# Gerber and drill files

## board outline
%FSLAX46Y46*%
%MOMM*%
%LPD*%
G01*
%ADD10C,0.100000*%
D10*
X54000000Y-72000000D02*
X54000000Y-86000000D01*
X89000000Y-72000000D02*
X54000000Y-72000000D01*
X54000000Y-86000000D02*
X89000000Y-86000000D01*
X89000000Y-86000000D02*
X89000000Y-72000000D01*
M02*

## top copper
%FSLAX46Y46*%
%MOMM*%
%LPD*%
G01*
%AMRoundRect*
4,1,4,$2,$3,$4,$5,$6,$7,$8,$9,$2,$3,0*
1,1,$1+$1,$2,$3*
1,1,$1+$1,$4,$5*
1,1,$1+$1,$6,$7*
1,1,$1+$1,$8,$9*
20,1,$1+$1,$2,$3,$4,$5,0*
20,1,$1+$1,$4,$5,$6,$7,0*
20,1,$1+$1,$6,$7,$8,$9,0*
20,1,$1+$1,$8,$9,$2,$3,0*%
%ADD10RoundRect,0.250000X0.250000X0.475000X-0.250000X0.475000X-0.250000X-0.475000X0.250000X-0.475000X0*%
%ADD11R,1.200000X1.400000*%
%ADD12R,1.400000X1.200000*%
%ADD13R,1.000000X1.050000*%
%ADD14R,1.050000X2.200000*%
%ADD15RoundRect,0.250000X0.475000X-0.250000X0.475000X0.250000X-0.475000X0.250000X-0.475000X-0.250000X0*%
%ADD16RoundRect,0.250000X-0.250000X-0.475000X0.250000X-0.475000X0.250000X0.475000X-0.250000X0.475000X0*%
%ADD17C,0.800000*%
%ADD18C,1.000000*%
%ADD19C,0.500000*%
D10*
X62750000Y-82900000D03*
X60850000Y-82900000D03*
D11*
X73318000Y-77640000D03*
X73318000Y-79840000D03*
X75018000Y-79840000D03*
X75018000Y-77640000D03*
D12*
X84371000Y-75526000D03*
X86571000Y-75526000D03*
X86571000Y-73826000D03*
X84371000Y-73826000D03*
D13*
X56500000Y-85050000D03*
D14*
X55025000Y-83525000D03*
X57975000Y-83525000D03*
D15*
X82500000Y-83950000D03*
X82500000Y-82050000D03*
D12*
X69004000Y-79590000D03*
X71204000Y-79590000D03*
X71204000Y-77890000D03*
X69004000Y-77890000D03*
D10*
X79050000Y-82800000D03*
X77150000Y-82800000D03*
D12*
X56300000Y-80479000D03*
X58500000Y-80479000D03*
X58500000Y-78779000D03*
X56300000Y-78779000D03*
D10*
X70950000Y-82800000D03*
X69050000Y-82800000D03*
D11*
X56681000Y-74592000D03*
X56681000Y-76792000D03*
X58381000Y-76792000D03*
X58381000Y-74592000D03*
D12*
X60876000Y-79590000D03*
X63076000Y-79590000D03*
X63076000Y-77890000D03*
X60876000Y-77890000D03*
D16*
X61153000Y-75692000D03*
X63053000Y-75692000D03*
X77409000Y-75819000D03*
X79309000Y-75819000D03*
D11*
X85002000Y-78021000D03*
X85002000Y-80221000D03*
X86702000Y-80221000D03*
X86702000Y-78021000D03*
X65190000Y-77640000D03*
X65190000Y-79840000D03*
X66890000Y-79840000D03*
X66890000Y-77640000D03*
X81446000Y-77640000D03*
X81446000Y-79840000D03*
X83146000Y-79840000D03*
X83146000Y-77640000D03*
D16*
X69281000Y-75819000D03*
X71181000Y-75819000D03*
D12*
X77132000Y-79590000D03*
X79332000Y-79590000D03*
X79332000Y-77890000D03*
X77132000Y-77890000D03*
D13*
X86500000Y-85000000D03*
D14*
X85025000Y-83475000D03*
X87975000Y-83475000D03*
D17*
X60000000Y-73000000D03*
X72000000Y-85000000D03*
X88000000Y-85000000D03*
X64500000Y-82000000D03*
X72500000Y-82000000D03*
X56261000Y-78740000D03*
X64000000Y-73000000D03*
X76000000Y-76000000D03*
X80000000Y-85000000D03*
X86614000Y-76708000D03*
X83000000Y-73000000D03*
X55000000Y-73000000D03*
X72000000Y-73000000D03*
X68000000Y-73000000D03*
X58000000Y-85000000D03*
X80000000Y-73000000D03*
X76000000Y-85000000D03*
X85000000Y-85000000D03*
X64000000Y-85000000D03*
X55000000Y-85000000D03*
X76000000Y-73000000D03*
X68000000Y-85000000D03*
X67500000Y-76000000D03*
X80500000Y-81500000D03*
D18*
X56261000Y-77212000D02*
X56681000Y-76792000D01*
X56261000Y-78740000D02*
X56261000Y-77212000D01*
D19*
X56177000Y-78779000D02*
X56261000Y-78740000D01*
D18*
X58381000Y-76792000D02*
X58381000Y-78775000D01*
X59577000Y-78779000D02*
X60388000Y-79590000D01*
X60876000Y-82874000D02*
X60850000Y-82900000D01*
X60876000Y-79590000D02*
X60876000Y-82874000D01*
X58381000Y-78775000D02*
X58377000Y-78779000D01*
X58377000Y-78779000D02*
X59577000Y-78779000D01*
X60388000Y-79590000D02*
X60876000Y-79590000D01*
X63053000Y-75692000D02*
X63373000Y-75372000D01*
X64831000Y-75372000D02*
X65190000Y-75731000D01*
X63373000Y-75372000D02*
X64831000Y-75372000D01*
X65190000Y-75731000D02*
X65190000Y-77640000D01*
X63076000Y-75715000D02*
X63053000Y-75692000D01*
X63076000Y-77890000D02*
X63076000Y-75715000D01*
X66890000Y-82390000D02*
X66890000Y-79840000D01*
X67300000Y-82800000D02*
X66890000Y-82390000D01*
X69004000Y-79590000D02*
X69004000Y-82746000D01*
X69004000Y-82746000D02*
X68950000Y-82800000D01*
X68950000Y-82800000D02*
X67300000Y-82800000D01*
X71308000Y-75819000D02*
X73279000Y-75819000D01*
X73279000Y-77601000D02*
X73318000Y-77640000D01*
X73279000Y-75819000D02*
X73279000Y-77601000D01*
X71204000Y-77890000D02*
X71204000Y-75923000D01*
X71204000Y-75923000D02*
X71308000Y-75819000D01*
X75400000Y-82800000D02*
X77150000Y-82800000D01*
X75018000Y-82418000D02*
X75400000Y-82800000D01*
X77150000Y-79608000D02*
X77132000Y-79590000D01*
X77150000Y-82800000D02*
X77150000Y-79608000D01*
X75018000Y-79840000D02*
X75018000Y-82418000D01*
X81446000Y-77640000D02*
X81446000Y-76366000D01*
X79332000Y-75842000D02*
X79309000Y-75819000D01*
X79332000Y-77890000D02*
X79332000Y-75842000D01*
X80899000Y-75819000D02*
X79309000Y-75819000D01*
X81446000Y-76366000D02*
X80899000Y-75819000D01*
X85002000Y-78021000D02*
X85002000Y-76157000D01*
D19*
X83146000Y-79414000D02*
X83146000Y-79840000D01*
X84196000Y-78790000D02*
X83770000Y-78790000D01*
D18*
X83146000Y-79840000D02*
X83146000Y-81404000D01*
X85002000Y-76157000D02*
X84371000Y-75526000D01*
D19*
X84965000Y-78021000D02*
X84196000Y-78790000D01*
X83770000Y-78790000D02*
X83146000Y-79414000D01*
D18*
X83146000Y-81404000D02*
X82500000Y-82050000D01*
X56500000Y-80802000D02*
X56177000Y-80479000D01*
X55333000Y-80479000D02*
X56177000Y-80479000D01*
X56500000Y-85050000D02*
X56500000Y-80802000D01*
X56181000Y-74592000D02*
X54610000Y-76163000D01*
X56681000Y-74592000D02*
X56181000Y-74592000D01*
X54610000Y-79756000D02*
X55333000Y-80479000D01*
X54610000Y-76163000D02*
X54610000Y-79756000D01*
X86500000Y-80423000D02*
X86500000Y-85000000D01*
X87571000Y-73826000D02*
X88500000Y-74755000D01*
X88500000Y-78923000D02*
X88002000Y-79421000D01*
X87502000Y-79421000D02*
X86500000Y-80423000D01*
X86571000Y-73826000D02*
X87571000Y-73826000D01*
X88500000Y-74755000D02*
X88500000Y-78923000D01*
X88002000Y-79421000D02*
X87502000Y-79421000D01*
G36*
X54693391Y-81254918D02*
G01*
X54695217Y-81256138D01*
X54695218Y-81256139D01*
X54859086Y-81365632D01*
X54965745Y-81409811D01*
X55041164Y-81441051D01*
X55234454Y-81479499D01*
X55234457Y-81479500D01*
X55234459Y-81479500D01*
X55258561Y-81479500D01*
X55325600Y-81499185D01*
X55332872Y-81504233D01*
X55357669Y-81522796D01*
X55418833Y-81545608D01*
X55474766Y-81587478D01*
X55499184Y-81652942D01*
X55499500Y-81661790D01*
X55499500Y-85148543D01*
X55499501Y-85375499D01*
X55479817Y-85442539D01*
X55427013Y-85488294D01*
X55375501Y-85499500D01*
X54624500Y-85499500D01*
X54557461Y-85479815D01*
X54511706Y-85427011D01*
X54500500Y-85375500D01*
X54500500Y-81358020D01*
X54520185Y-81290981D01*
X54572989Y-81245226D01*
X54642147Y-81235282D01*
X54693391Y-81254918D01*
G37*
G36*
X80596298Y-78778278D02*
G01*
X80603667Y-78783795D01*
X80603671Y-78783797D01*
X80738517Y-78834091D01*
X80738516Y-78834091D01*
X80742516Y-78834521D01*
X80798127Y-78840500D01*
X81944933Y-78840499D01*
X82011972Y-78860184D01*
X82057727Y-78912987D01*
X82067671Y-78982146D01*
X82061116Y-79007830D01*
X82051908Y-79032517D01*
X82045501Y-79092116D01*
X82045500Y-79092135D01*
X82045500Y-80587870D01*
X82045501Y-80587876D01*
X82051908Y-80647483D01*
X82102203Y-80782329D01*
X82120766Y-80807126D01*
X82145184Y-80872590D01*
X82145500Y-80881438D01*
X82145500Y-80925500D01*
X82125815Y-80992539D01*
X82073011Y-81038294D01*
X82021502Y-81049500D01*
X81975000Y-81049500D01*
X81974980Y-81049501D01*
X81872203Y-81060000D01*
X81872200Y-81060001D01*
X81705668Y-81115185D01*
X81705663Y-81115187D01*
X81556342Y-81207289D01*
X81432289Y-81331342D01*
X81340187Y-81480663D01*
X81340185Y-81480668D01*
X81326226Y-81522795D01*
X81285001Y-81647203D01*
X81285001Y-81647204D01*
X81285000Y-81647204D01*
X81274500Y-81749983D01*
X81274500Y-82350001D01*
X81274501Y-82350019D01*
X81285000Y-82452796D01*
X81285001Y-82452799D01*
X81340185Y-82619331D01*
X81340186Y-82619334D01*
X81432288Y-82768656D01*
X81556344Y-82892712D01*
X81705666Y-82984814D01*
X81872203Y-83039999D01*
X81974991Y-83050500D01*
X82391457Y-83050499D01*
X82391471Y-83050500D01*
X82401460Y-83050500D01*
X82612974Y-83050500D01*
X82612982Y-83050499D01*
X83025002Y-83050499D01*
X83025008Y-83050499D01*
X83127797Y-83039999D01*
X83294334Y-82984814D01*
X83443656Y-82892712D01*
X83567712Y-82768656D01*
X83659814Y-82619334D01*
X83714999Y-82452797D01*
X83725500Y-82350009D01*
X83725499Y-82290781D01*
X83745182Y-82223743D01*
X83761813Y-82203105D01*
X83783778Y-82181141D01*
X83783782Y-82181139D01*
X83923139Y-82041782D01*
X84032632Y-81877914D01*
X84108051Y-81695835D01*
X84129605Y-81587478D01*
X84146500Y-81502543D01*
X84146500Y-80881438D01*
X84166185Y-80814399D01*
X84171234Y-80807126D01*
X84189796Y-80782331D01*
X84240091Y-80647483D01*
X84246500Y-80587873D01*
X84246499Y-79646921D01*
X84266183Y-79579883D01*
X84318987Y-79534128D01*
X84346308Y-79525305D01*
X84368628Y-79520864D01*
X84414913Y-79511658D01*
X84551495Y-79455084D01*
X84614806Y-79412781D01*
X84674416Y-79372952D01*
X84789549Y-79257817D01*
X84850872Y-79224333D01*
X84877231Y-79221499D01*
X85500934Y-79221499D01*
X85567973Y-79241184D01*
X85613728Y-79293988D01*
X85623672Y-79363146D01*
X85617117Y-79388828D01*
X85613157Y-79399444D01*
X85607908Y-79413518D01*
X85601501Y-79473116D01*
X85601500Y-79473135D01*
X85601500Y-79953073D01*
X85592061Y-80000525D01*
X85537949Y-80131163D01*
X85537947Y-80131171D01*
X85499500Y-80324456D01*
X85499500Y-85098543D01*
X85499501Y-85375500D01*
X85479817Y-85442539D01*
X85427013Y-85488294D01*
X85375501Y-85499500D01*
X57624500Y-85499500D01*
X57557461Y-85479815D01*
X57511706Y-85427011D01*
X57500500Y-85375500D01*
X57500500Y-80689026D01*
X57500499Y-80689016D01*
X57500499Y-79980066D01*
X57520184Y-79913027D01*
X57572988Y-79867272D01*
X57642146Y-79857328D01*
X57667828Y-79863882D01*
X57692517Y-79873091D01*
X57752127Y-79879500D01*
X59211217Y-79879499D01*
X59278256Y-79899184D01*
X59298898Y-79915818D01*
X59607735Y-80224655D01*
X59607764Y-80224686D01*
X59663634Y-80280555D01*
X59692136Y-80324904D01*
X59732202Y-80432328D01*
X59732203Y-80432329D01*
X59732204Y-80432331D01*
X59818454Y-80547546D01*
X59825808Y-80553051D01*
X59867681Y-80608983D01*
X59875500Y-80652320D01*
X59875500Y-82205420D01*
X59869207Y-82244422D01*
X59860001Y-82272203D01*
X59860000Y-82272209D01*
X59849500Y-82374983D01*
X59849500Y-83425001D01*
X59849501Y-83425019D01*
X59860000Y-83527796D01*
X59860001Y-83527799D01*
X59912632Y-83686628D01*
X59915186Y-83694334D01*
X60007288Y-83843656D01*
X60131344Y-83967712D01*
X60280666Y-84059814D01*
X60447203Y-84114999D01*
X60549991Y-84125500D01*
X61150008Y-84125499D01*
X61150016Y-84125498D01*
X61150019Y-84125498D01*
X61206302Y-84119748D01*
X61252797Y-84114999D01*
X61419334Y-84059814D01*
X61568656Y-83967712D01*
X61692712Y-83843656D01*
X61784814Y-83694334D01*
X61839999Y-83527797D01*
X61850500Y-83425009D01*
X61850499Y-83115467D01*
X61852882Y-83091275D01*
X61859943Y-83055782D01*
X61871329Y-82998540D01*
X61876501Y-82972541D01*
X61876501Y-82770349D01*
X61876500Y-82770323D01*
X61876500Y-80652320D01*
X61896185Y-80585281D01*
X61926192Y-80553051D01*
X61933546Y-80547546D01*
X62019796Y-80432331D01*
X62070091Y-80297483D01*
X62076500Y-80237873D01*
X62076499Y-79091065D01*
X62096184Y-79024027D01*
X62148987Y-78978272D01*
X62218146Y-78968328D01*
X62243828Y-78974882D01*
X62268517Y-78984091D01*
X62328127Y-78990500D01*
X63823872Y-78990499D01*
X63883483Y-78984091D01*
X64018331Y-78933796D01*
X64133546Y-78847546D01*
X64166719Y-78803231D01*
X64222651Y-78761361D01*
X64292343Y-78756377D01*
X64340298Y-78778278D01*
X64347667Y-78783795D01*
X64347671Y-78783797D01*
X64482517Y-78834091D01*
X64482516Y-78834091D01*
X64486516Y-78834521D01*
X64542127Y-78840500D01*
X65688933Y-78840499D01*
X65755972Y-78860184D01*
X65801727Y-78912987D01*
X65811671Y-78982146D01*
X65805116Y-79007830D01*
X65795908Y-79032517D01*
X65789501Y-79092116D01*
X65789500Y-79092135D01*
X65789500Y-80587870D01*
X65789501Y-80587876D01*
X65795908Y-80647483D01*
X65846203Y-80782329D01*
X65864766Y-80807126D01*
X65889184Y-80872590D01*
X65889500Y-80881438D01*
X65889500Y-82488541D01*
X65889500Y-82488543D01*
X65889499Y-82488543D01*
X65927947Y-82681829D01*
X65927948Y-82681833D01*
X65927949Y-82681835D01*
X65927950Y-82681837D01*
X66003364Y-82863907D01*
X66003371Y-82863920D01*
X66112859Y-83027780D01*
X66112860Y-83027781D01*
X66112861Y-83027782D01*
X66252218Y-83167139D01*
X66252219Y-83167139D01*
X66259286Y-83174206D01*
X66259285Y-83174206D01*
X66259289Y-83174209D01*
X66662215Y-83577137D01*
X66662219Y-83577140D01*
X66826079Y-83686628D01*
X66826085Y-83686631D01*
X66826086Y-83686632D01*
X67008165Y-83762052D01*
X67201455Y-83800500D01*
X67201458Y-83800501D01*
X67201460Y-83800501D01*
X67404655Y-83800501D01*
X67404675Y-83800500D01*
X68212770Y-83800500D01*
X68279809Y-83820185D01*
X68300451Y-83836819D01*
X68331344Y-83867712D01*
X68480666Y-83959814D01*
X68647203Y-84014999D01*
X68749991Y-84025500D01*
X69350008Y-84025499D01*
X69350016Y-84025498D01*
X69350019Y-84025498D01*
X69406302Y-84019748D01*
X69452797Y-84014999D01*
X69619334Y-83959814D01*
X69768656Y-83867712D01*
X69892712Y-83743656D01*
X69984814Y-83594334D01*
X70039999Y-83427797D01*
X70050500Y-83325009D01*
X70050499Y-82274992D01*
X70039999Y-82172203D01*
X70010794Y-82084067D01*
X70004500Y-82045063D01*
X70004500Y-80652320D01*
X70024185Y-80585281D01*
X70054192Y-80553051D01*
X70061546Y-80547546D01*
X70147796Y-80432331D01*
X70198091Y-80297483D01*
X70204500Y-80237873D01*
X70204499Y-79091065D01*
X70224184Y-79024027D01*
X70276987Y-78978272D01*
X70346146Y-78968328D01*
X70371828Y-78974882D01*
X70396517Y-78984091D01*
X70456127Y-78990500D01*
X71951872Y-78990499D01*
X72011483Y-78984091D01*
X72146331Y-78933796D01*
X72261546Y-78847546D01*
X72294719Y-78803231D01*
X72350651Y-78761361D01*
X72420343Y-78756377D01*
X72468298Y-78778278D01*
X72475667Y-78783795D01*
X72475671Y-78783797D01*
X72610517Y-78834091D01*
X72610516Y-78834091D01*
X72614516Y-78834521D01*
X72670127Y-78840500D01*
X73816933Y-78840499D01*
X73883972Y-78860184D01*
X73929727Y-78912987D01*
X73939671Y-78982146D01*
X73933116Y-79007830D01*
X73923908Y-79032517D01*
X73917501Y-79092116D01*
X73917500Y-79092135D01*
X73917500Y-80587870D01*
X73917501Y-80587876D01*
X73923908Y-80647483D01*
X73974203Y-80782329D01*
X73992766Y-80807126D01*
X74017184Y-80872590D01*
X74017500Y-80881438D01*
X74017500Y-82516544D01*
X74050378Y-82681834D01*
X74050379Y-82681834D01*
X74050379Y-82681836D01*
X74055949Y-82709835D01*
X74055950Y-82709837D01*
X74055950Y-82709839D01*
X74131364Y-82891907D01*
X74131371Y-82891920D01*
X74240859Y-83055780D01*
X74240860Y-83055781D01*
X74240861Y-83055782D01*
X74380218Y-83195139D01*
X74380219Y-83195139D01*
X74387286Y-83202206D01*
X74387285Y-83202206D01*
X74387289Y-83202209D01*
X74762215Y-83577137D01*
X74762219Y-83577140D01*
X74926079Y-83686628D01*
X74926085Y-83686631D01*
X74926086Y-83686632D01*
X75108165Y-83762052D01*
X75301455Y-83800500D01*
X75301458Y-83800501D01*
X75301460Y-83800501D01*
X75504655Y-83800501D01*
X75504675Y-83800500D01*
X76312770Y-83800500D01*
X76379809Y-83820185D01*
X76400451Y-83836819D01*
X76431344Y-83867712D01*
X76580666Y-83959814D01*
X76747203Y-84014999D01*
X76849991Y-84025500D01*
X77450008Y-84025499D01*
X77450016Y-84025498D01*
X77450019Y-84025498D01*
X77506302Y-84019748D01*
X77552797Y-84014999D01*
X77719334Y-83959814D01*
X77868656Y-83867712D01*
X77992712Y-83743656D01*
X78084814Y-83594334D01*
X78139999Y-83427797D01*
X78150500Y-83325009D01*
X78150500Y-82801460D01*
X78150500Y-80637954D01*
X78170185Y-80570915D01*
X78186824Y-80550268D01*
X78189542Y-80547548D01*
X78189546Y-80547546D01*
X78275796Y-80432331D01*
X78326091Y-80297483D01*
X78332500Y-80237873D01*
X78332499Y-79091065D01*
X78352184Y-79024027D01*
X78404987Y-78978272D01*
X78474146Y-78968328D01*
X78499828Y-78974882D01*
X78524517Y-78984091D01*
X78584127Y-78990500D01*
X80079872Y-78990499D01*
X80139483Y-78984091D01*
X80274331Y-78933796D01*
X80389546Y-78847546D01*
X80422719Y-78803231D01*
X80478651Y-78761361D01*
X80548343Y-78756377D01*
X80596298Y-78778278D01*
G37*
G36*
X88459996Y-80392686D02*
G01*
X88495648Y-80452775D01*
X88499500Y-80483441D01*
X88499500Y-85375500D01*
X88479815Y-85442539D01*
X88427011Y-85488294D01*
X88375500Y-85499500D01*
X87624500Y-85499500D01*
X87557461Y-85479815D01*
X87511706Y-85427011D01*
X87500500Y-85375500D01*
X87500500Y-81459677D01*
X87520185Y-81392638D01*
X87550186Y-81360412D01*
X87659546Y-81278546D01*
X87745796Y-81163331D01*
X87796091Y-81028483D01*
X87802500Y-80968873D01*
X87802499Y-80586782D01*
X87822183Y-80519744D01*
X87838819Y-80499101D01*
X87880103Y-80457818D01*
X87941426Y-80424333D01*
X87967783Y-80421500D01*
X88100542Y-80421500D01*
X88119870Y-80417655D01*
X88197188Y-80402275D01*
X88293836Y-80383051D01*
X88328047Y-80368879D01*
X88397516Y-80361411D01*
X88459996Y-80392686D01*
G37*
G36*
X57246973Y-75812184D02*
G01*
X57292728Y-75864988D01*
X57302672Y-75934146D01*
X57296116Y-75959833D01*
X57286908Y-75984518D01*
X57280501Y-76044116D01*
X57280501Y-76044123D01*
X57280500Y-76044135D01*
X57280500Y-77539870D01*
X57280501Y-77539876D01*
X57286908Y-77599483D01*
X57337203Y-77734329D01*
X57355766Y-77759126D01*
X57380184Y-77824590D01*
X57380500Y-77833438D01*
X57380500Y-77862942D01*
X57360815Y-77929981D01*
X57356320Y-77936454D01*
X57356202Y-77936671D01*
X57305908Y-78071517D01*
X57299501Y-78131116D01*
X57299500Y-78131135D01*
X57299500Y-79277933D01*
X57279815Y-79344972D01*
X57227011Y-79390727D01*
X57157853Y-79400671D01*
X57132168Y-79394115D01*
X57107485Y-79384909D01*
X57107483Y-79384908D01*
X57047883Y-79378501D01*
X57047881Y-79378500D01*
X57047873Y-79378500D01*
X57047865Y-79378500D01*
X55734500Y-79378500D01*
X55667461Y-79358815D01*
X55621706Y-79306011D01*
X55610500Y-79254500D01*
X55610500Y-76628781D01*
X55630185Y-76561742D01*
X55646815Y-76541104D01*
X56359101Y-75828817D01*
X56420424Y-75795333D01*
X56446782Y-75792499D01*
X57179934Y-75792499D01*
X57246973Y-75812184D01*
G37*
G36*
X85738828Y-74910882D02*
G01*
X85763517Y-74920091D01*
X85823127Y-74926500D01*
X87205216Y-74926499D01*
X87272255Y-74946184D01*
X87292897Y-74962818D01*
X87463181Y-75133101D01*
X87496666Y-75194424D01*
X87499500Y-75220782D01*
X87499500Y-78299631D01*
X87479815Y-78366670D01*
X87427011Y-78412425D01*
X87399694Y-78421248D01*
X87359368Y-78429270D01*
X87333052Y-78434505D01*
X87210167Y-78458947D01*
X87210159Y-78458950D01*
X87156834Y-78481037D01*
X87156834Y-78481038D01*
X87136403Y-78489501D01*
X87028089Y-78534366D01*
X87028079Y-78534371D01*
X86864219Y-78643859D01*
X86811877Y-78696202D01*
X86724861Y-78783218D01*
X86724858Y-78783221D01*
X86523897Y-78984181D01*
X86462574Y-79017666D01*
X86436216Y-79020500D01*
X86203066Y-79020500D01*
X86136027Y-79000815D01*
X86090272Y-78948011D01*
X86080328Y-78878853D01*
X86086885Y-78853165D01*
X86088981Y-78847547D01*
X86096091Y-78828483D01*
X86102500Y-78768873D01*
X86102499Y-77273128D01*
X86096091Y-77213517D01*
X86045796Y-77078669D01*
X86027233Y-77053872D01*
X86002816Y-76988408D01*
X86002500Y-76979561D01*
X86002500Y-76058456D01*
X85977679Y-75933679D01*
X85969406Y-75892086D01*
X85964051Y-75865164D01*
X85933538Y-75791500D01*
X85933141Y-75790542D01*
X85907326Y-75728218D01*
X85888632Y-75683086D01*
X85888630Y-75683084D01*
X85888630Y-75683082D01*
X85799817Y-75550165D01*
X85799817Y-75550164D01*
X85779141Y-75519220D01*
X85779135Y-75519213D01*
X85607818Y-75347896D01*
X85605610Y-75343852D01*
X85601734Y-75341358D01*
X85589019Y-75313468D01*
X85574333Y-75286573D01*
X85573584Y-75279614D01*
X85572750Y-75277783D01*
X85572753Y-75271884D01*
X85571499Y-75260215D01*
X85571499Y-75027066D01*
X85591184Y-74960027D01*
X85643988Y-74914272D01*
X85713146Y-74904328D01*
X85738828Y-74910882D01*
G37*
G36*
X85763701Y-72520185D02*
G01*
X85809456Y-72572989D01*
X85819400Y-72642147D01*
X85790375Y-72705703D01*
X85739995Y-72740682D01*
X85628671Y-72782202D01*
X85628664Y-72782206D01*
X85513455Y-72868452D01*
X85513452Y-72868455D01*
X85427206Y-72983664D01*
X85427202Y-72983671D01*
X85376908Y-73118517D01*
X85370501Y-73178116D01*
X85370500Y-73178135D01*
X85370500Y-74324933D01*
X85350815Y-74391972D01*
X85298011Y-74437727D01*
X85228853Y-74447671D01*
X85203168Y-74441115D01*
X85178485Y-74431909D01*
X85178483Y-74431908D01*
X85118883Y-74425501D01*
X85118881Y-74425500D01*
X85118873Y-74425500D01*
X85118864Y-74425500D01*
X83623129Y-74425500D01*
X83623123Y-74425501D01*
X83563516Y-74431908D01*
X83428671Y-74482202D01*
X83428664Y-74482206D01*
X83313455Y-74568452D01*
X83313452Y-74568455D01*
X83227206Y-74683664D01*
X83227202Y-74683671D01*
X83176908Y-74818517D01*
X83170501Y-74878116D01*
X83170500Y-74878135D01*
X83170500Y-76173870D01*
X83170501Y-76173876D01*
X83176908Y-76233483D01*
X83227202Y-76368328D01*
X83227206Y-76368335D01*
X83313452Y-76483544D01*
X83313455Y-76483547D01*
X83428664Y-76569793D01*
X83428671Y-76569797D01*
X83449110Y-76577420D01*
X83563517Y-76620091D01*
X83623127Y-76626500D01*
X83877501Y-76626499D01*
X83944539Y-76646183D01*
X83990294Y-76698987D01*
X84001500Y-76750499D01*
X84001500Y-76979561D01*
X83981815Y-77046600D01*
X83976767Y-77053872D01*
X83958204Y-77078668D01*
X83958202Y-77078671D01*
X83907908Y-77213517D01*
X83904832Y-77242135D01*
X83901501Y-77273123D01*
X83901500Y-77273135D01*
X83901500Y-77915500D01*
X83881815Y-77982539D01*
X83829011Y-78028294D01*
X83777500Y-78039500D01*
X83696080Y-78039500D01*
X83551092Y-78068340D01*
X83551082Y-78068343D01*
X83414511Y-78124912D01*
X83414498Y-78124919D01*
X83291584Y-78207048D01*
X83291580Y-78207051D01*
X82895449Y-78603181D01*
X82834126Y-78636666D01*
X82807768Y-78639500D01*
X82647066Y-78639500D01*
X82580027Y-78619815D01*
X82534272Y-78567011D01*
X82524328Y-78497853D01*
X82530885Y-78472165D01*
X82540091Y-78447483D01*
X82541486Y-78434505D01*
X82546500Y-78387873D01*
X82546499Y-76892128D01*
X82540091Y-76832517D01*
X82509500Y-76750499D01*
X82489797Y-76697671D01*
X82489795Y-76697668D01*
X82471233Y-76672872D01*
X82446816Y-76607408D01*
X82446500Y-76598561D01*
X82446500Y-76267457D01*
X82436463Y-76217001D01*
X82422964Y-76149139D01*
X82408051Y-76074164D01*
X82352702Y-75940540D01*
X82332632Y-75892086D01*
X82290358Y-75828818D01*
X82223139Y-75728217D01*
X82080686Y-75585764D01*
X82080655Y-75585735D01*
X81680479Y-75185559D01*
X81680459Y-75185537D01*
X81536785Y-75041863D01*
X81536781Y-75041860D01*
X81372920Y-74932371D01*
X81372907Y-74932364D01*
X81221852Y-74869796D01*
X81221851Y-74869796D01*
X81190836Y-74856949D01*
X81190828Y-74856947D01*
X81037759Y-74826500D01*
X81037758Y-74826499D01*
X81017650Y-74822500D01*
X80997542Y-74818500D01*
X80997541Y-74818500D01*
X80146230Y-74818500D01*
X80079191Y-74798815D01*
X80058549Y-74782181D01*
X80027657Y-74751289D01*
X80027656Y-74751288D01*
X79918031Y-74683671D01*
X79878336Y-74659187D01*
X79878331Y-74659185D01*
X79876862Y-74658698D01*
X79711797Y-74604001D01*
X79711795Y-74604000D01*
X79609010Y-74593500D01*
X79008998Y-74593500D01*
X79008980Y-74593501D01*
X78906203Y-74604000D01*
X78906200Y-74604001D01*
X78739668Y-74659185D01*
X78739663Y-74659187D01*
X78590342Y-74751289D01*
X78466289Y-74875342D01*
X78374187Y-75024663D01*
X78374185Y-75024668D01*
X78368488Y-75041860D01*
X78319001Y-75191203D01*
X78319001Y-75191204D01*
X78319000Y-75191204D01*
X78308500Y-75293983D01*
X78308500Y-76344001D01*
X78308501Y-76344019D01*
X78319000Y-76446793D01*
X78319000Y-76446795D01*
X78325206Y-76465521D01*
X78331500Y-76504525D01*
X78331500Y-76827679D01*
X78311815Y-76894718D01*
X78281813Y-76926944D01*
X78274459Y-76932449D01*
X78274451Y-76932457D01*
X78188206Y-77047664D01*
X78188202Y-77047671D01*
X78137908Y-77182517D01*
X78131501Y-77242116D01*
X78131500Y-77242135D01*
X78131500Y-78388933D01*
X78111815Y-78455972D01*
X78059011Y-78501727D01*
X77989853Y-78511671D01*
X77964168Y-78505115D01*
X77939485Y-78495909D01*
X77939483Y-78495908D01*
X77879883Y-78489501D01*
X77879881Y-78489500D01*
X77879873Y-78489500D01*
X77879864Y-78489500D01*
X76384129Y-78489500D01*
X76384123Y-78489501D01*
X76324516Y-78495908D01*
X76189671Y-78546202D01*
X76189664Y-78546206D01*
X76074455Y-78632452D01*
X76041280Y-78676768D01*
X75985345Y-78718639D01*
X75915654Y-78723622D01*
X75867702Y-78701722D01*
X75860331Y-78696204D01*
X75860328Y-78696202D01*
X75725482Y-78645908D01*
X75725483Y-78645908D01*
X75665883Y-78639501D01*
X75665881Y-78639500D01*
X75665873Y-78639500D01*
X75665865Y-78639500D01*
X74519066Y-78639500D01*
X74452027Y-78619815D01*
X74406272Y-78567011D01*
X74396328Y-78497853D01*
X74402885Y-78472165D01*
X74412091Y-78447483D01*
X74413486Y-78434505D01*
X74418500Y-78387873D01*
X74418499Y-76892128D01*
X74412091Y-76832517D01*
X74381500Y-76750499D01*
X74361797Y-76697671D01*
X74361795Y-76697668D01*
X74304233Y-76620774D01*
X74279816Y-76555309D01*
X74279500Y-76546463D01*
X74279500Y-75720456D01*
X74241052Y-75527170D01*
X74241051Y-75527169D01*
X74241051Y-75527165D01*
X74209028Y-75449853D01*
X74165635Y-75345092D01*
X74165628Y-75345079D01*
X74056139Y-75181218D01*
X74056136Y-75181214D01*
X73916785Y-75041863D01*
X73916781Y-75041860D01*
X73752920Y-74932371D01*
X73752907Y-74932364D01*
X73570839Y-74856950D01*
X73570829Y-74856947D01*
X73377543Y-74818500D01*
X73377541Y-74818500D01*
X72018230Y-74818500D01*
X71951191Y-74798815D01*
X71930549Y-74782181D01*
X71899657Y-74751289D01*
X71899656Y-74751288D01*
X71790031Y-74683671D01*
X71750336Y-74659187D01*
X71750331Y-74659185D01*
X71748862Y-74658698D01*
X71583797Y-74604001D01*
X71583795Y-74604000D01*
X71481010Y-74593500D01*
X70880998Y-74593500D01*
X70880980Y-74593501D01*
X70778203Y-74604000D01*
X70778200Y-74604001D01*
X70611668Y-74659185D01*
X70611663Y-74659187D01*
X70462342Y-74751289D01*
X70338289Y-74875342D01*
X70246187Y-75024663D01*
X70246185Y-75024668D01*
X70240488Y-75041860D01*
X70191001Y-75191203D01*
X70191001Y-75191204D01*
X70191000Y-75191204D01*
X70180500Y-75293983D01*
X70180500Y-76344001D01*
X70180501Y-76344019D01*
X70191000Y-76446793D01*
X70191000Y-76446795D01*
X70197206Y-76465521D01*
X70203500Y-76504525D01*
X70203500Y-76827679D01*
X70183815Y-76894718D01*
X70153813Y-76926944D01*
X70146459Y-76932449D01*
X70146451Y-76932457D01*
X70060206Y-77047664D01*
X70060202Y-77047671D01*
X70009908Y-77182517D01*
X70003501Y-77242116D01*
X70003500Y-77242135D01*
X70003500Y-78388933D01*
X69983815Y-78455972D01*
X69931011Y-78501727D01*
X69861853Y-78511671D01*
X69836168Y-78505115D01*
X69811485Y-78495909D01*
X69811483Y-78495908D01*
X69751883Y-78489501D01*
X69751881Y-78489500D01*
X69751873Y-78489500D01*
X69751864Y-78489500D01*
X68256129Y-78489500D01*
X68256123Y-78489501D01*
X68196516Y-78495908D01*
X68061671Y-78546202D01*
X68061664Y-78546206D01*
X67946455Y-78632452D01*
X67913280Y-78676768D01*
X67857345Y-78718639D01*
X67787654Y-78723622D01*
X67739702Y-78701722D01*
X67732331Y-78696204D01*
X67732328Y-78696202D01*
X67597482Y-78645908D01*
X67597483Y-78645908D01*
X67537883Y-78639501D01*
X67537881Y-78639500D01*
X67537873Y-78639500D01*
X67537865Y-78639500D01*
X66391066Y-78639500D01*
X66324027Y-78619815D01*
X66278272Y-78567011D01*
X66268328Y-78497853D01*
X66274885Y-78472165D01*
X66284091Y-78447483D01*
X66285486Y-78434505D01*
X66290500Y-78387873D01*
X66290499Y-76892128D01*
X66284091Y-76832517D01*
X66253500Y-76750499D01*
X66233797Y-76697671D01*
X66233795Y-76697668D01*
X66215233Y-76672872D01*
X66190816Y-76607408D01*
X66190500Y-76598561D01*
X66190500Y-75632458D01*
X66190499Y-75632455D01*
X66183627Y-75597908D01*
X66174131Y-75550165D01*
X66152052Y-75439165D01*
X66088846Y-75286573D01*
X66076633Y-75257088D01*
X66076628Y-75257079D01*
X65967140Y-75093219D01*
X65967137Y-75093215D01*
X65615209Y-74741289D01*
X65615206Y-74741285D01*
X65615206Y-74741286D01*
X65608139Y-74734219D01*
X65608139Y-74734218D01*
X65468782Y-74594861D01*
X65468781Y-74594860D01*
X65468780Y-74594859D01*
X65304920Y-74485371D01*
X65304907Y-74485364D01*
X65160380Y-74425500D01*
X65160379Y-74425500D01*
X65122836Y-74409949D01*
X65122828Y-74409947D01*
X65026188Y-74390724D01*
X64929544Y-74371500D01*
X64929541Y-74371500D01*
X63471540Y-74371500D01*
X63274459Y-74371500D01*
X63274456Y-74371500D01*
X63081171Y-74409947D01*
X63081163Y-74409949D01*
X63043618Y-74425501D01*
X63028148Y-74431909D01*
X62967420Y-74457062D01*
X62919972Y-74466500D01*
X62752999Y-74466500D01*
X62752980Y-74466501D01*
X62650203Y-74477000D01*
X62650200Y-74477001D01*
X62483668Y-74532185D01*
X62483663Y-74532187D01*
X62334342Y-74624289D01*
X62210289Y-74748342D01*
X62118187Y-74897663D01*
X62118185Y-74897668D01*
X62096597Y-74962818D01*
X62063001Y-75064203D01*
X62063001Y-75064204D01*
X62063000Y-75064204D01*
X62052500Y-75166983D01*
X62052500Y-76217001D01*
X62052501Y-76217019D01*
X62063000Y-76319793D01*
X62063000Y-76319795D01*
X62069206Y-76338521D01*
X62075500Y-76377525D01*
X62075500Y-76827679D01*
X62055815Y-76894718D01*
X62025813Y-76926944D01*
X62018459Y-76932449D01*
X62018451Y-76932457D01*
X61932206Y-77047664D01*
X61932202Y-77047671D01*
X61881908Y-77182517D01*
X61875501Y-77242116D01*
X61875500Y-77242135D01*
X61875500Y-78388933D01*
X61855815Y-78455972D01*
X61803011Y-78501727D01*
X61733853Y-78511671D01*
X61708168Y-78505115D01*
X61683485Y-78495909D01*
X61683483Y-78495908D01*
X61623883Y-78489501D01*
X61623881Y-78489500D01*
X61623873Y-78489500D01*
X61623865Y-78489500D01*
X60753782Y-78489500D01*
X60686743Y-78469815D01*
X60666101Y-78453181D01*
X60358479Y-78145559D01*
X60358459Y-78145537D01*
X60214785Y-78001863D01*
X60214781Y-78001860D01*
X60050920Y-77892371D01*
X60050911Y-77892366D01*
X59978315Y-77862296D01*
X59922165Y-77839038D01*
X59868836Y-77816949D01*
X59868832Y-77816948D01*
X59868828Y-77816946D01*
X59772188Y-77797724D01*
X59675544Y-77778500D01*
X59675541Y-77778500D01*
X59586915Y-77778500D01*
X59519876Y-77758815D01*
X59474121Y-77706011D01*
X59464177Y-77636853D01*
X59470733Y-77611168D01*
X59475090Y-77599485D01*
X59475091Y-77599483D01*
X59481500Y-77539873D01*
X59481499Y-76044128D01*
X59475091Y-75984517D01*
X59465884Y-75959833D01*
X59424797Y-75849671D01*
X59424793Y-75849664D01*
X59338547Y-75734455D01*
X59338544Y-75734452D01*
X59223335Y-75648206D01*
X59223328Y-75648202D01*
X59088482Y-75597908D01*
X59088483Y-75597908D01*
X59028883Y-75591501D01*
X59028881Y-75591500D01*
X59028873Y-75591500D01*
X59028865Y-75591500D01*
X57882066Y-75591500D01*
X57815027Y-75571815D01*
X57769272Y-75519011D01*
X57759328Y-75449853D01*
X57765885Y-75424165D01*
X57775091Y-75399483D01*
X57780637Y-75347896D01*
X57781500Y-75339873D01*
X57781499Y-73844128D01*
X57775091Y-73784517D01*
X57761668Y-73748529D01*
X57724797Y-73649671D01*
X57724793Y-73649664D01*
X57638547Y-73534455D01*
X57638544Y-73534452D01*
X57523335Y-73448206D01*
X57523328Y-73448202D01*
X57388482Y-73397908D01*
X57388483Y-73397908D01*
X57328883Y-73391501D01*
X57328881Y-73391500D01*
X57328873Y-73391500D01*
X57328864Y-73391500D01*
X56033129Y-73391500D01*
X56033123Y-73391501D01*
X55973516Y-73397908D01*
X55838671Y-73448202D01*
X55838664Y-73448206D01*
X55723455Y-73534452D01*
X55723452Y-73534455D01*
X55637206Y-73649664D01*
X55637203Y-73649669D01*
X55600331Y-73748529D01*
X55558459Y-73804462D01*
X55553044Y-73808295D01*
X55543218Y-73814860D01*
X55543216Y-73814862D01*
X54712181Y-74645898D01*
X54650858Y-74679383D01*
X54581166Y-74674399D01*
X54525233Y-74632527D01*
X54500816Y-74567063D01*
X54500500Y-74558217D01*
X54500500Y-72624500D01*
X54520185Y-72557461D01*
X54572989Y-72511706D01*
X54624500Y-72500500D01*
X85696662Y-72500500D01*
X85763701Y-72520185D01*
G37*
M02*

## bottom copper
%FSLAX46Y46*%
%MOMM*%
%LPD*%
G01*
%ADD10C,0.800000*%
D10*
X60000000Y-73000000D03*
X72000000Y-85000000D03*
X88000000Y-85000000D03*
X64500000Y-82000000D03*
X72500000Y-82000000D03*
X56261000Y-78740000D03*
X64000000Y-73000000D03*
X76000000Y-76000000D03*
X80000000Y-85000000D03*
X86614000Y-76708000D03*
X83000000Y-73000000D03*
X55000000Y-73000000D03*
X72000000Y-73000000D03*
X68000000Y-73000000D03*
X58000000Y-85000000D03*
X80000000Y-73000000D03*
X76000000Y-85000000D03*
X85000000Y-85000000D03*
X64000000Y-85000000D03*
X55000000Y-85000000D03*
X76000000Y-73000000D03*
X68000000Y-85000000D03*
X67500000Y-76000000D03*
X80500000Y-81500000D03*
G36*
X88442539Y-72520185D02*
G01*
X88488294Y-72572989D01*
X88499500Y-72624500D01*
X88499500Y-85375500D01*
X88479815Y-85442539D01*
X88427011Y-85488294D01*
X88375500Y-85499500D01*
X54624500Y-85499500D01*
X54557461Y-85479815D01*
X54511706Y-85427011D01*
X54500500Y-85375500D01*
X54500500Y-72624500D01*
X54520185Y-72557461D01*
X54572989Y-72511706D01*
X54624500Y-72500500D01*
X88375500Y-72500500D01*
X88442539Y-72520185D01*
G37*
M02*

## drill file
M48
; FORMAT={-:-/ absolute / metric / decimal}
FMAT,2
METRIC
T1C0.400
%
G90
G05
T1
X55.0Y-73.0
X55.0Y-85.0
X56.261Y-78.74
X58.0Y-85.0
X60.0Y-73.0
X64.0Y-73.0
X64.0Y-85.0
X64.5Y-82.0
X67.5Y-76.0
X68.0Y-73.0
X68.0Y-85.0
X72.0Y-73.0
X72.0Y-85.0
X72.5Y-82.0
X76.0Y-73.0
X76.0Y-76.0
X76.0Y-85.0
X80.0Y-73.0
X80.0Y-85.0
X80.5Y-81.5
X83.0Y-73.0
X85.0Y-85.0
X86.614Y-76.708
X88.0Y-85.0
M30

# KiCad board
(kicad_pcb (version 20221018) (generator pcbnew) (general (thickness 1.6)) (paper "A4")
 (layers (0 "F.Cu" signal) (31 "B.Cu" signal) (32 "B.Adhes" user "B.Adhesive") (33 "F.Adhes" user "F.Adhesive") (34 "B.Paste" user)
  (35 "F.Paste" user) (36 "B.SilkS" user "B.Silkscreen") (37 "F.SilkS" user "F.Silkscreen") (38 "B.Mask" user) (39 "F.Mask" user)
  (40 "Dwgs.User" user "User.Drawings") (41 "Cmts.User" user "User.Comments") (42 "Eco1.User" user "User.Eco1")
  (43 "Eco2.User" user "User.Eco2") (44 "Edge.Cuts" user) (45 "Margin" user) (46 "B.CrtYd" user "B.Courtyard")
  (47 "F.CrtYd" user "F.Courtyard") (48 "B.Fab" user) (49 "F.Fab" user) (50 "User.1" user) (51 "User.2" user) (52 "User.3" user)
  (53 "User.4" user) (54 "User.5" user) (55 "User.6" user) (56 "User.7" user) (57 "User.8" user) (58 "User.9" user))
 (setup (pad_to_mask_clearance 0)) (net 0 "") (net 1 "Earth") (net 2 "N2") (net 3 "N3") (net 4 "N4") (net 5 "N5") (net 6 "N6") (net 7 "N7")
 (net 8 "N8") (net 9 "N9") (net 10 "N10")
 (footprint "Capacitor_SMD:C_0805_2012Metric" (layer "F.Cu") (at 61.8 82.9 180)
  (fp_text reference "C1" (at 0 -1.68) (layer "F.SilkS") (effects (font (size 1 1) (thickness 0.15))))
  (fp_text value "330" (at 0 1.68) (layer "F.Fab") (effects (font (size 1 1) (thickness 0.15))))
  (pad "1" smd roundrect (at -0.95 0 180) (size 1 1.45) (layers "F.Cu" "F.Paste" "F.Mask") (roundrect_rratio 0.25) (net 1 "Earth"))
  (pad "2" smd roundrect (at 0.95 0 180) (size 1 1.45) (layers "F.Cu" "F.Paste" "F.Mask") (roundrect_rratio 0.25) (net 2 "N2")))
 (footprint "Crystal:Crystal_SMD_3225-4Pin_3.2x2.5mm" (layer "F.Cu") (at 74.168 78.74 -90)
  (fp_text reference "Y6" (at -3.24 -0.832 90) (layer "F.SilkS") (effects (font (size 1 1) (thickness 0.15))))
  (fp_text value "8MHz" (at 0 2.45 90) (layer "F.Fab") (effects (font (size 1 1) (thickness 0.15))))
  (pad "1" smd rect (at -1.1 0.85 270) (size 1.4 1.2) (layers "F.Cu" "F.Paste" "F.Mask") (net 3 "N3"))
  (pad "2" smd rect (at 1.1 0.85 270) (size 1.4 1.2) (layers "F.Cu" "F.Paste" "F.Mask") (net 1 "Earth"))
  (pad "3" smd rect (at 1.1 -0.85 270) (size 1.4 1.2) (layers "F.Cu" "F.Paste" "F.Mask") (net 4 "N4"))
  (pad "4" smd rect (at -1.1 -0.85 270) (size 1.4 1.2) (layers "F.Cu" "F.Paste" "F.Mask") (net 1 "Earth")))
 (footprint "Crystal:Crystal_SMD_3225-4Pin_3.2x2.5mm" (layer "F.Cu") (at 85.471 74.676)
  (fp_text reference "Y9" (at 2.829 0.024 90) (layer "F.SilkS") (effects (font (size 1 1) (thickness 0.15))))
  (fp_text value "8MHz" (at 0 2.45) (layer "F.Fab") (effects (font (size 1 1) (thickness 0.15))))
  (pad "1" smd rect (at -1.1 0.85) (size 1.4 1.2) (layers "F.Cu" "F.Paste" "F.Mask") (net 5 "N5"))
  (pad "2" smd rect (at 1.1 0.85) (size 1.4 1.2) (layers "F.Cu" "F.Paste" "F.Mask") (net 1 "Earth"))
  (pad "3" smd rect (at 1.1 -0.85) (size 1.4 1.2) (layers "F.Cu" "F.Paste" "F.Mask") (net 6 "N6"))
  (pad "4" smd rect (at -1.1 -0.85) (size 1.4 1.2) (layers "F.Cu" "F.Paste" "F.Mask") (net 1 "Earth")))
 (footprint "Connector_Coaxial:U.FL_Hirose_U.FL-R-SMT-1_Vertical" (layer "F.Cu") (at 56.5 84 90)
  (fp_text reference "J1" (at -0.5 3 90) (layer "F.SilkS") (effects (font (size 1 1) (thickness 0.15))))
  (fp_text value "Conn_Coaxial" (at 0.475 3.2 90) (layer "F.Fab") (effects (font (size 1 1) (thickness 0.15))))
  (pad "1" smd rect (at -1.05 0 90) (size 1.05 1) (layers "F.Cu" "F.Paste" "F.Mask") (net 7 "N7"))
  (pad "2" smd rect (at 0.475 -1.475 90) (size 2.2 1.05) (layers "F.Cu" "F.Paste" "F.Mask") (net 1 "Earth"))
  (pad "2" smd rect (at 0.475 1.475 90) (size 2.2 1.05) (layers "F.Cu" "F.Paste" "F.Mask") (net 1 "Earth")))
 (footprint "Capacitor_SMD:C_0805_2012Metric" (layer "F.Cu") (at 82.5 83 90)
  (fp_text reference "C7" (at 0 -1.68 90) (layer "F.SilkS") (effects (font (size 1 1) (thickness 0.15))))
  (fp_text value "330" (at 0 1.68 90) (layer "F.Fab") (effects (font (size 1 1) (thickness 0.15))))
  (pad "1" smd roundrect (at -0.95 0 90) (size 1 1.45) (layers "F.Cu" "F.Paste" "F.Mask") (roundrect_rratio 0.25) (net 1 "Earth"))
  (pad "2" smd roundrect (at 0.95 0 90) (size 1 1.45) (layers "F.Cu" "F.Paste" "F.Mask") (roundrect_rratio 0.25) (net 5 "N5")))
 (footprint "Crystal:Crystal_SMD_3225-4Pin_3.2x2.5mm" (layer "F.Cu") (at 70.104 78.74)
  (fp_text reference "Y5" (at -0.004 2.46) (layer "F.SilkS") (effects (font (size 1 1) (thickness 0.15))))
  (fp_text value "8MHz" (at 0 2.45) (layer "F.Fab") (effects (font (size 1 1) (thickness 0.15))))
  (pad "1" smd rect (at -1.1 0.85) (size 1.4 1.2) (layers "F.Cu" "F.Paste" "F.Mask") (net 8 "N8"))
  (pad "2" smd rect (at 1.1 0.85) (size 1.4 1.2) (layers "F.Cu" "F.Paste" "F.Mask") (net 1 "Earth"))
  (pad "3" smd rect (at 1.1 -0.85) (size 1.4 1.2) (layers "F.Cu" "F.Paste" "F.Mask") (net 3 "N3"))
  (pad "4" smd rect (at -1.1 -0.85) (size 1.4 1.2) (layers "F.Cu" "F.Paste" "F.Mask") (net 1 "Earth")))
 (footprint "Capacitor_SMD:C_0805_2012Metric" (layer "F.Cu") (at 78.1 82.8 180)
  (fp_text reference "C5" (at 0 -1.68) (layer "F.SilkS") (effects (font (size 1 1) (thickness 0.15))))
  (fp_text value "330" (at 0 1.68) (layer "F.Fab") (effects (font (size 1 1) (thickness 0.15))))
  (pad "1" smd roundrect (at -0.95 0 180) (size 1 1.45) (layers "F.Cu" "F.Paste" "F.Mask") (roundrect_rratio 0.25) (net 1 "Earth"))
  (pad "2" smd roundrect (at 0.95 0 180) (size 1 1.45) (layers "F.Cu" "F.Paste" "F.Mask") (roundrect_rratio 0.25) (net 4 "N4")))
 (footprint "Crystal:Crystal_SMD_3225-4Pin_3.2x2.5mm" (layer "F.Cu") (at 57.4 79.629)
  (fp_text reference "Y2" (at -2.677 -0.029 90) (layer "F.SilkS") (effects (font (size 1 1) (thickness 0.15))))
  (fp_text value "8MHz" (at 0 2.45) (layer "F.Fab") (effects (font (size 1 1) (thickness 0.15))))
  (pad "1" smd rect (at -1.1 0.85) (size 1.4 1.2) (layers "F.Cu" "F.Paste" "F.Mask") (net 7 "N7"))
  (pad "2" smd rect (at 1.1 0.85) (size 1.4 1.2) (layers "F.Cu" "F.Paste" "F.Mask") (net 1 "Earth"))
  (pad "3" smd rect (at 1.1 -0.85) (size 1.4 1.2) (layers "F.Cu" "F.Paste" "F.Mask") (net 2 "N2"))
  (pad "4" smd rect (at -1.1 -0.85) (size 1.4 1.2) (layers "F.Cu" "F.Paste" "F.Mask") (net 1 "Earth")))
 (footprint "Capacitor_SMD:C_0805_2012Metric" (layer "F.Cu") (at 70 82.8 180)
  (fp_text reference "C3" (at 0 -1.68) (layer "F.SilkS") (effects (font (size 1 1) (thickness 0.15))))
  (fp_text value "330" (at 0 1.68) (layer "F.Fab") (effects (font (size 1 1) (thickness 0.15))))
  (pad "1" smd roundrect (at -0.95 0 180) (size 1 1.45) (layers "F.Cu" "F.Paste" "F.Mask") (roundrect_rratio 0.25) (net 1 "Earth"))
  (pad "2" smd roundrect (at 0.95 0 180) (size 1 1.45) (layers "F.Cu" "F.Paste" "F.Mask") (roundrect_rratio 0.25) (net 8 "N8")))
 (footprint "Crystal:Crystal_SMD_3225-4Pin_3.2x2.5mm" (layer "F.Cu") (at 57.531 75.692 -90)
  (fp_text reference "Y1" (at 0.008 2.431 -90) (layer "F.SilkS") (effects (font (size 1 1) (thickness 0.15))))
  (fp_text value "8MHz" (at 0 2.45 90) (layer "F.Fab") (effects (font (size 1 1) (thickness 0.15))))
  (pad "1" smd rect (at -1.1 0.85 270) (size 1.4 1.2) (layers "F.Cu" "F.Paste" "F.Mask") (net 7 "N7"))
  (pad "2" smd rect (at 1.1 0.85 270) (size 1.4 1.2) (layers "F.Cu" "F.Paste" "F.Mask") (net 1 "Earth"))
  (pad "3" smd rect (at 1.1 -0.85 270) (size 1.4 1.2) (layers "F.Cu" "F.Paste" "F.Mask") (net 2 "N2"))
  (pad "4" smd rect (at -1.1 -0.85 270) (size 1.4 1.2) (layers "F.Cu" "F.Paste" "F.Mask") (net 1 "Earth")))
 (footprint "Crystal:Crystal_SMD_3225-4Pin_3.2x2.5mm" (layer "F.Cu") (at 61.976 78.74)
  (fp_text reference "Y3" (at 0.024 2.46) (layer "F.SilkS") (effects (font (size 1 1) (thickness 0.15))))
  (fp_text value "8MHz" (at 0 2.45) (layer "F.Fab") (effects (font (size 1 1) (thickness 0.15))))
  (pad "1" smd rect (at -1.1 0.85) (size 1.4 1.2) (layers "F.Cu" "F.Paste" "F.Mask") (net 2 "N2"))
  (pad "2" smd rect (at 1.1 0.85) (size 1.4 1.2) (layers "F.Cu" "F.Paste" "F.Mask") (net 1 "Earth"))
  (pad "3" smd rect (at 1.1 -0.85) (size 1.4 1.2) (layers "F.Cu" "F.Paste" "F.Mask") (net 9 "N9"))
  (pad "4" smd rect (at -1.1 -0.85) (size 1.4 1.2) (layers "F.Cu" "F.Paste" "F.Mask") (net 1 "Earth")))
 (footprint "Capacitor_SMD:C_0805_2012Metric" (layer "F.Cu") (at 62.103 75.692)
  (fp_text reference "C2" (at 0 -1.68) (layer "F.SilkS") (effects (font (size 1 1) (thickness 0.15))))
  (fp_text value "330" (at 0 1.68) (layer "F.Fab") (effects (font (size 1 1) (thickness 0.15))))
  (pad "1" smd roundrect (at -0.95 0) (size 1 1.45) (layers "F.Cu" "F.Paste" "F.Mask") (roundrect_rratio 0.25) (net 1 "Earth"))
  (pad "2" smd roundrect (at 0.95 0) (size 1 1.45) (layers "F.Cu" "F.Paste" "F.Mask") (roundrect_rratio 0.25) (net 9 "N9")))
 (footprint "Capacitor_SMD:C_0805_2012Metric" (layer "F.Cu") (at 78.359 75.819)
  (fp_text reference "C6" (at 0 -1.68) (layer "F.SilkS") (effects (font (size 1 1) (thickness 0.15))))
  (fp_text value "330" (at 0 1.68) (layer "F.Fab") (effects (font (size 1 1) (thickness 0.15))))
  (pad "1" smd roundrect (at -0.95 0) (size 1 1.45) (layers "F.Cu" "F.Paste" "F.Mask") (roundrect_rratio 0.25) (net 1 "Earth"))
  (pad "2" smd roundrect (at 0.95 0) (size 1 1.45) (layers "F.Cu" "F.Paste" "F.Mask") (roundrect_rratio 0.25) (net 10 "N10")))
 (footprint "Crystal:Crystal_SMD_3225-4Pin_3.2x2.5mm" (layer "F.Cu") (at 85.852 79.121 -90)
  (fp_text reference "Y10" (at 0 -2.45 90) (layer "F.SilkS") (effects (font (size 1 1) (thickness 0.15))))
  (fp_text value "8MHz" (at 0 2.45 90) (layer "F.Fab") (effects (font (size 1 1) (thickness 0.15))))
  (pad "1" smd rect (at -1.1 0.85 270) (size 1.4 1.2) (layers "F.Cu" "F.Paste" "F.Mask") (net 5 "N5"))
  (pad "2" smd rect (at 1.1 0.85 270) (size 1.4 1.2) (layers "F.Cu" "F.Paste" "F.Mask") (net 1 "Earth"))
  (pad "3" smd rect (at 1.1 -0.85 270) (size 1.4 1.2) (layers "F.Cu" "F.Paste" "F.Mask") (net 6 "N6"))
  (pad "4" smd rect (at -1.1 -0.85 270) (size 1.4 1.2) (layers "F.Cu" "F.Paste" "F.Mask") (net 1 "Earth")))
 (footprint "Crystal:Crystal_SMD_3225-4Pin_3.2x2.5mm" (layer "F.Cu") (at 66.04 78.74 -90)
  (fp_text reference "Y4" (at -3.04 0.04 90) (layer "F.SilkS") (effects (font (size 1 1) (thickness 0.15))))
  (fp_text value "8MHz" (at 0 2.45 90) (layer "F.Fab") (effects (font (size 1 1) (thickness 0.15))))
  (pad "1" smd rect (at -1.1 0.85 270) (size 1.4 1.2) (layers "F.Cu" "F.Paste" "F.Mask") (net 9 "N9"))
  (pad "2" smd rect (at 1.1 0.85 270) (size 1.4 1.2) (layers "F.Cu" "F.Paste" "F.Mask") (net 1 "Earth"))
  (pad "3" smd rect (at 1.1 -0.85 270) (size 1.4 1.2) (layers "F.Cu" "F.Paste" "F.Mask") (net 8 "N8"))
  (pad "4" smd rect (at -1.1 -0.85 270) (size 1.4 1.2) (layers "F.Cu" "F.Paste" "F.Mask") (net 1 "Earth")))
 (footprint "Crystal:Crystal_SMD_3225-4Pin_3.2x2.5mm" (layer "F.Cu") (at 82.296 78.74 -90)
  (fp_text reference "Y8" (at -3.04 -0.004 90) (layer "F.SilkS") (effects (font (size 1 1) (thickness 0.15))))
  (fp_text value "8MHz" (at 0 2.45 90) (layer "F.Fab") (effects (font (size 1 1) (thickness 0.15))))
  (pad "1" smd rect (at -1.1 0.85 270) (size 1.4 1.2) (layers "F.Cu" "F.Paste" "F.Mask") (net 10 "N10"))
  (pad "2" smd rect (at 1.1 0.85 270) (size 1.4 1.2) (layers "F.Cu" "F.Paste" "F.Mask") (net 1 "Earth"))
  (pad "3" smd rect (at 1.1 -0.85 270) (size 1.4 1.2) (layers "F.Cu" "F.Paste" "F.Mask") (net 5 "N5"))
  (pad "4" smd rect (at -1.1 -0.85 270) (size 1.4 1.2) (layers "F.Cu" "F.Paste" "F.Mask") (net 1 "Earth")))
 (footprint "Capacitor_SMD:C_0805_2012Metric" (layer "F.Cu") (at 70.231 75.819)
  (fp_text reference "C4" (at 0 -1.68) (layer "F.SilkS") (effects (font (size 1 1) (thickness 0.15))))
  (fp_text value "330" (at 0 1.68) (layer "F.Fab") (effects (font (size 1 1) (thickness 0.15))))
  (pad "1" smd roundrect (at -0.95 0) (size 1 1.45) (layers "F.Cu" "F.Paste" "F.Mask") (roundrect_rratio 0.25) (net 1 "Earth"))
  (pad "2" smd roundrect (at 0.95 0) (size 1 1.45) (layers "F.Cu" "F.Paste" "F.Mask") (roundrect_rratio 0.25) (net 3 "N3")))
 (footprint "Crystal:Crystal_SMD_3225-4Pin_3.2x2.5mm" (layer "F.Cu") (at 78.232 78.74)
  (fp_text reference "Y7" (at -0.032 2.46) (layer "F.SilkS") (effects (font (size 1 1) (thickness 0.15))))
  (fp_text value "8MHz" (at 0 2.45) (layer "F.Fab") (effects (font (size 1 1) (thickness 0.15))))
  (pad "1" smd rect (at -1.1 0.85) (size 1.4 1.2) (layers "F.Cu" "F.Paste" "F.Mask") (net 4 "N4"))
  (pad "2" smd rect (at 1.1 0.85) (size 1.4 1.2) (layers "F.Cu" "F.Paste" "F.Mask") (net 1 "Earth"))
  (pad "3" smd rect (at 1.1 -0.85) (size 1.4 1.2) (layers "F.Cu" "F.Paste" "F.Mask") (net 10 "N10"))
  (pad "4" smd rect (at -1.1 -0.85) (size 1.4 1.2) (layers "F.Cu" "F.Paste" "F.Mask") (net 1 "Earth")))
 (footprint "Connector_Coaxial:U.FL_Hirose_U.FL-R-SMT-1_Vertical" (layer "F.Cu") (at 86.5 83.95 90)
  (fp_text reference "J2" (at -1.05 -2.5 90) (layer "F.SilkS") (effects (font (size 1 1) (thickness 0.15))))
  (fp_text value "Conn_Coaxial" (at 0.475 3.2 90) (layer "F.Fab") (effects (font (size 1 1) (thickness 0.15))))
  (pad "1" smd rect (at -1.05 0 90) (size 1.05 1) (layers "F.Cu" "F.Paste" "F.Mask") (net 6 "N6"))
  (pad "2" smd rect (at 0.475 -1.475 90) (size 2.2 1.05) (layers "F.Cu" "F.Paste" "F.Mask") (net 1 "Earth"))
  (pad "2" smd rect (at 0.475 1.475 90) (size 2.2 1.05) (layers "F.Cu" "F.Paste" "F.Mask") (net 1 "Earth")))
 (gr_line (start 54 72) (end 54 86) (stroke (width 0.1) (type default)) (layer "Edge.Cuts"))
 (gr_line (start 89 72) (end 54 72) (stroke (width 0.1) (type default)) (layer "Edge.Cuts"))
 (gr_line (start 54 86) (end 89 86) (stroke (width 0.1) (type default)) (layer "Edge.Cuts"))
 (gr_line (start 89 86) (end 89 72) (stroke (width 0.1) (type default)) (layer "Edge.Cuts"))
 (segment (start 56.261 77.212) (end 56.681 76.792) (width 1) (layer "F.Cu") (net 1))
 (segment (start 56.261 78.74) (end 56.261 77.212) (width 1) (layer "F.Cu") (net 1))
 (segment (start 56.177 78.779) (end 56.261 78.74) (width 0.5) (layer "F.Cu") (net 1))
 (via (at 60 73) (size 0.8) (drill 0.4) (layers "F.Cu" "B.Cu") (free) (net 1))
 (via (at 72 85) (size 0.8) (drill 0.4) (layers "F.Cu" "B.Cu") (free) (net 1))
 (via (at 88 85) (size 0.8) (drill 0.4) (layers "F.Cu" "B.Cu") (free) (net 1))
 (via (at 64.5 82) (size 0.8) (drill 0.4) (layers "F.Cu" "B.Cu") (free) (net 1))
 (via (at 72.5 82) (size 0.8) (drill 0.4) (layers "F.Cu" "B.Cu") (free) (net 1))
 (via (at 56.261 78.74) (size 0.8) (drill 0.4) (layers "F.Cu" "B.Cu") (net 1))
 (via (at 64 73) (size 0.8) (drill 0.4) (layers "F.Cu" "B.Cu") (free) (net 1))
 (via (at 76 76) (size 0.8) (drill 0.4) (layers "F.Cu" "B.Cu") (free) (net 1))
 (via (at 80 85) (size 0.8) (drill 0.4) (layers "F.Cu" "B.Cu") (free) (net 1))
 (via (at 86.614 76.708) (size 0.8) (drill 0.4) (layers "F.Cu" "B.Cu") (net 1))
 (via (at 83 73) (size 0.8) (drill 0.4) (layers "F.Cu" "B.Cu") (free) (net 1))
 (via (at 55 73) (size 0.8) (drill 0.4) (layers "F.Cu" "B.Cu") (free) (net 1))
 (via (at 72 73) (size 0.8) (drill 0.4) (layers "F.Cu" "B.Cu") (free) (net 1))
 (via (at 68 73) (size 0.8) (drill 0.4) (layers "F.Cu" "B.Cu") (free) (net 1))
 (via (at 58 85) (size 0.8) (drill 0.4) (layers "F.Cu" "B.Cu") (free) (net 1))
 (via (at 80 73) (size 0.8) (drill 0.4) (layers "F.Cu" "B.Cu") (free) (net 1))
 (via (at 76 85) (size 0.8) (drill 0.4) (layers "F.Cu" "B.Cu") (free) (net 1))
 (via (at 85 85) (size 0.8) (drill 0.4) (layers "F.Cu" "B.Cu") (free) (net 1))
 (via (at 64 85) (size 0.8) (drill 0.4) (layers "F.Cu" "B.Cu") (free) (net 1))
 (via (at 55 85) (size 0.8) (drill 0.4) (layers "F.Cu" "B.Cu") (free) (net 1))
 (via (at 76 73) (size 0.8) (drill 0.4) (layers "F.Cu" "B.Cu") (free) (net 1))
 (via (at 68 85) (size 0.8) (drill 0.4) (layers "F.Cu" "B.Cu") (free) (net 1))
 (via (at 67.5 76) (size 0.8) (drill 0.4) (layers "F.Cu" "B.Cu") (free) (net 1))
 (via (at 80.5 81.5) (size 0.8) (drill 0.4) (layers "F.Cu" "B.Cu") (free) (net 1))
 (segment (start 58.381 76.792) (end 58.381 78.775) (width 1) (layer "F.Cu") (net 2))
 (segment (start 59.577 78.779) (end 60.388 79.59) (width 1) (layer "F.Cu") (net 2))
 (segment (start 60.876 82.874) (end 60.85 82.9) (width 1) (layer "F.Cu") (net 2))
 (segment (start 60.876 79.59) (end 60.876 82.874) (width 1) (layer "F.Cu") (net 2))
 (segment (start 58.381 78.775) (end 58.377 78.779) (width 1) (layer "F.Cu") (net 2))
 (segment (start 58.377 78.779) (end 59.577 78.779) (width 1) (layer "F.Cu") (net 2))
 (segment (start 60.388 79.59) (end 60.876 79.59) (width 1) (layer "F.Cu") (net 2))
 (segment (start 63.053 75.692) (end 63.373 75.372) (width 1) (layer "F.Cu") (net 9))
 (segment (start 64.831 75.372) (end 65.19 75.731) (width 1) (layer "F.Cu") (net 9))
 (segment (start 63.373 75.372) (end 64.831 75.372) (width 1) (layer "F.Cu") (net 9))
 (segment (start 65.19 75.731) (end 65.19 77.64) (width 1) (layer "F.Cu") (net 9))
 (segment (start 63.076 75.715) (end 63.053 75.692) (width 1) (layer "F.Cu") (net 9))
 (segment (start 63.076 77.89) (end 63.076 75.715) (width 1) (layer "F.Cu") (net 9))
 (segment (start 66.89 82.39) (end 66.89 79.84) (width 1) (layer "F.Cu") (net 8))
 (segment (start 67.3 82.8) (end 66.89 82.39) (width 1) (layer "F.Cu") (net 8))
 (segment (start 69.004 79.59) (end 69.004 82.746) (width 1) (layer "F.Cu") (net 8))
 (segment (start 69.004 82.746) (end 68.95 82.8) (width 1) (layer "F.Cu") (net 8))
 (segment (start 68.95 82.8) (end 67.3 82.8) (width 1) (layer "F.Cu") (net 8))
 (segment (start 71.308 75.819) (end 73.279 75.819) (width 1) (layer "F.Cu") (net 3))
 (segment (start 73.279 77.601) (end 73.318 77.64) (width 1) (layer "F.Cu") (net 3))
 (segment (start 73.279 75.819) (end 73.279 77.601) (width 1) (layer "F.Cu") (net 3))
 (segment (start 71.204 77.89) (end 71.204 75.923) (width 1) (layer "F.Cu") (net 3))
 (segment (start 71.204 75.923) (end 71.308 75.819) (width 1) (layer "F.Cu") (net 3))
 (segment (start 75.4 82.8) (end 77.15 82.8) (width 1) (layer "F.Cu") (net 4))
 (segment (start 75.018 82.418) (end 75.4 82.8) (width 1) (layer "F.Cu") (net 4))
 (segment (start 77.15 79.608) (end 77.132 79.59) (width 1) (layer "F.Cu") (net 4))
 (segment (start 77.15 82.8) (end 77.15 79.608) (width 1) (layer "F.Cu") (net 4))
 (segment (start 75.018 79.84) (end 75.018 82.418) (width 1) (layer "F.Cu") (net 4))
 (segment (start 81.446 77.64) (end 81.446 76.366) (width 1) (layer "F.Cu") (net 10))
 (segment (start 79.332 75.842) (end 79.309 75.819) (width 1) (layer "F.Cu") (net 10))
 (segment (start 79.332 77.89) (end 79.332 75.842) (width 1) (layer "F.Cu") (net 10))
 (segment (start 80.899 75.819) (end 79.309 75.819) (width 1) (layer "F.Cu") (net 10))
 (segment (start 81.446 76.366) (end 80.899 75.819) (width 1) (layer "F.Cu") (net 10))
 (segment (start 85.002 78.021) (end 85.002 76.157) (width 1) (layer "F.Cu") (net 5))
 (segment (start 83.146 79.414) (end 83.146 79.84) (width 0.5) (layer "F.Cu") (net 5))
 (segment (start 84.196 78.79) (end 83.77 78.79) (width 0.5) (layer "F.Cu") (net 5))
 (segment (start 83.146 79.84) (end 83.146 81.404) (width 1) (layer "F.Cu") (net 5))
 (segment (start 85.002 76.157) (end 84.371 75.526) (width 1) (layer "F.Cu") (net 5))
 (segment (start 84.965 78.021) (end 84.196 78.79) (width 0.5) (layer "F.Cu") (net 5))
 (segment (start 83.77 78.79) (end 83.146 79.414) (width 0.5) (layer "F.Cu") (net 5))
 (segment (start 83.146 81.404) (end 82.5 82.05) (width 1) (layer "F.Cu") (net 5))
 (segment (start 56.5 80.802) (end 56.177 80.479) (width 1) (layer "F.Cu") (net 7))
 (segment (start 55.333 80.479) (end 56.177 80.479) (width 1) (layer "F.Cu") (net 7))
 (segment (start 56.5 85.05) (end 56.5 80.802) (width 1) (layer "F.Cu") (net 7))
 (segment (start 56.181 74.592) (end 54.61 76.163) (width 1) (layer "F.Cu") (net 7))
 (segment (start 56.681 74.592) (end 56.181 74.592) (width 1) (layer "F.Cu") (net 7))
 (segment (start 54.61 79.756) (end 55.333 80.479) (width 1) (layer "F.Cu") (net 7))
 (segment (start 54.61 76.163) (end 54.61 79.756) (width 1) (layer "F.Cu") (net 7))
 (segment (start 86.5 80.423) (end 86.5 85) (width 1) (layer "F.Cu") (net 6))
 (segment (start 87.571 73.826) (end 88.5 74.755) (width 1) (layer "F.Cu") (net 6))
 (segment (start 88.5 78.923) (end 88.002 79.421) (width 1) (layer "F.Cu") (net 6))
 (segment (start 87.502 79.421) (end 86.5 80.423) (width 1) (layer "F.Cu") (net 6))
 (segment (start 86.571 73.826) (end 87.571 73.826) (width 1) (layer "F.Cu") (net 6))
 (segment (start 88.5 74.755) (end 88.5 78.923) (width 1) (layer "F.Cu") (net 6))
 (segment (start 88.002 79.421) (end 87.502 79.421) (width 1) (layer "F.Cu") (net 6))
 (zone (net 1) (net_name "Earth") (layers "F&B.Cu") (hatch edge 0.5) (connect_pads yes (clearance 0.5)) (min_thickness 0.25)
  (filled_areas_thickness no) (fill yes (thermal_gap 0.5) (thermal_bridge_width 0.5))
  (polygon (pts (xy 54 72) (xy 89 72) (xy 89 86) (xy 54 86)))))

